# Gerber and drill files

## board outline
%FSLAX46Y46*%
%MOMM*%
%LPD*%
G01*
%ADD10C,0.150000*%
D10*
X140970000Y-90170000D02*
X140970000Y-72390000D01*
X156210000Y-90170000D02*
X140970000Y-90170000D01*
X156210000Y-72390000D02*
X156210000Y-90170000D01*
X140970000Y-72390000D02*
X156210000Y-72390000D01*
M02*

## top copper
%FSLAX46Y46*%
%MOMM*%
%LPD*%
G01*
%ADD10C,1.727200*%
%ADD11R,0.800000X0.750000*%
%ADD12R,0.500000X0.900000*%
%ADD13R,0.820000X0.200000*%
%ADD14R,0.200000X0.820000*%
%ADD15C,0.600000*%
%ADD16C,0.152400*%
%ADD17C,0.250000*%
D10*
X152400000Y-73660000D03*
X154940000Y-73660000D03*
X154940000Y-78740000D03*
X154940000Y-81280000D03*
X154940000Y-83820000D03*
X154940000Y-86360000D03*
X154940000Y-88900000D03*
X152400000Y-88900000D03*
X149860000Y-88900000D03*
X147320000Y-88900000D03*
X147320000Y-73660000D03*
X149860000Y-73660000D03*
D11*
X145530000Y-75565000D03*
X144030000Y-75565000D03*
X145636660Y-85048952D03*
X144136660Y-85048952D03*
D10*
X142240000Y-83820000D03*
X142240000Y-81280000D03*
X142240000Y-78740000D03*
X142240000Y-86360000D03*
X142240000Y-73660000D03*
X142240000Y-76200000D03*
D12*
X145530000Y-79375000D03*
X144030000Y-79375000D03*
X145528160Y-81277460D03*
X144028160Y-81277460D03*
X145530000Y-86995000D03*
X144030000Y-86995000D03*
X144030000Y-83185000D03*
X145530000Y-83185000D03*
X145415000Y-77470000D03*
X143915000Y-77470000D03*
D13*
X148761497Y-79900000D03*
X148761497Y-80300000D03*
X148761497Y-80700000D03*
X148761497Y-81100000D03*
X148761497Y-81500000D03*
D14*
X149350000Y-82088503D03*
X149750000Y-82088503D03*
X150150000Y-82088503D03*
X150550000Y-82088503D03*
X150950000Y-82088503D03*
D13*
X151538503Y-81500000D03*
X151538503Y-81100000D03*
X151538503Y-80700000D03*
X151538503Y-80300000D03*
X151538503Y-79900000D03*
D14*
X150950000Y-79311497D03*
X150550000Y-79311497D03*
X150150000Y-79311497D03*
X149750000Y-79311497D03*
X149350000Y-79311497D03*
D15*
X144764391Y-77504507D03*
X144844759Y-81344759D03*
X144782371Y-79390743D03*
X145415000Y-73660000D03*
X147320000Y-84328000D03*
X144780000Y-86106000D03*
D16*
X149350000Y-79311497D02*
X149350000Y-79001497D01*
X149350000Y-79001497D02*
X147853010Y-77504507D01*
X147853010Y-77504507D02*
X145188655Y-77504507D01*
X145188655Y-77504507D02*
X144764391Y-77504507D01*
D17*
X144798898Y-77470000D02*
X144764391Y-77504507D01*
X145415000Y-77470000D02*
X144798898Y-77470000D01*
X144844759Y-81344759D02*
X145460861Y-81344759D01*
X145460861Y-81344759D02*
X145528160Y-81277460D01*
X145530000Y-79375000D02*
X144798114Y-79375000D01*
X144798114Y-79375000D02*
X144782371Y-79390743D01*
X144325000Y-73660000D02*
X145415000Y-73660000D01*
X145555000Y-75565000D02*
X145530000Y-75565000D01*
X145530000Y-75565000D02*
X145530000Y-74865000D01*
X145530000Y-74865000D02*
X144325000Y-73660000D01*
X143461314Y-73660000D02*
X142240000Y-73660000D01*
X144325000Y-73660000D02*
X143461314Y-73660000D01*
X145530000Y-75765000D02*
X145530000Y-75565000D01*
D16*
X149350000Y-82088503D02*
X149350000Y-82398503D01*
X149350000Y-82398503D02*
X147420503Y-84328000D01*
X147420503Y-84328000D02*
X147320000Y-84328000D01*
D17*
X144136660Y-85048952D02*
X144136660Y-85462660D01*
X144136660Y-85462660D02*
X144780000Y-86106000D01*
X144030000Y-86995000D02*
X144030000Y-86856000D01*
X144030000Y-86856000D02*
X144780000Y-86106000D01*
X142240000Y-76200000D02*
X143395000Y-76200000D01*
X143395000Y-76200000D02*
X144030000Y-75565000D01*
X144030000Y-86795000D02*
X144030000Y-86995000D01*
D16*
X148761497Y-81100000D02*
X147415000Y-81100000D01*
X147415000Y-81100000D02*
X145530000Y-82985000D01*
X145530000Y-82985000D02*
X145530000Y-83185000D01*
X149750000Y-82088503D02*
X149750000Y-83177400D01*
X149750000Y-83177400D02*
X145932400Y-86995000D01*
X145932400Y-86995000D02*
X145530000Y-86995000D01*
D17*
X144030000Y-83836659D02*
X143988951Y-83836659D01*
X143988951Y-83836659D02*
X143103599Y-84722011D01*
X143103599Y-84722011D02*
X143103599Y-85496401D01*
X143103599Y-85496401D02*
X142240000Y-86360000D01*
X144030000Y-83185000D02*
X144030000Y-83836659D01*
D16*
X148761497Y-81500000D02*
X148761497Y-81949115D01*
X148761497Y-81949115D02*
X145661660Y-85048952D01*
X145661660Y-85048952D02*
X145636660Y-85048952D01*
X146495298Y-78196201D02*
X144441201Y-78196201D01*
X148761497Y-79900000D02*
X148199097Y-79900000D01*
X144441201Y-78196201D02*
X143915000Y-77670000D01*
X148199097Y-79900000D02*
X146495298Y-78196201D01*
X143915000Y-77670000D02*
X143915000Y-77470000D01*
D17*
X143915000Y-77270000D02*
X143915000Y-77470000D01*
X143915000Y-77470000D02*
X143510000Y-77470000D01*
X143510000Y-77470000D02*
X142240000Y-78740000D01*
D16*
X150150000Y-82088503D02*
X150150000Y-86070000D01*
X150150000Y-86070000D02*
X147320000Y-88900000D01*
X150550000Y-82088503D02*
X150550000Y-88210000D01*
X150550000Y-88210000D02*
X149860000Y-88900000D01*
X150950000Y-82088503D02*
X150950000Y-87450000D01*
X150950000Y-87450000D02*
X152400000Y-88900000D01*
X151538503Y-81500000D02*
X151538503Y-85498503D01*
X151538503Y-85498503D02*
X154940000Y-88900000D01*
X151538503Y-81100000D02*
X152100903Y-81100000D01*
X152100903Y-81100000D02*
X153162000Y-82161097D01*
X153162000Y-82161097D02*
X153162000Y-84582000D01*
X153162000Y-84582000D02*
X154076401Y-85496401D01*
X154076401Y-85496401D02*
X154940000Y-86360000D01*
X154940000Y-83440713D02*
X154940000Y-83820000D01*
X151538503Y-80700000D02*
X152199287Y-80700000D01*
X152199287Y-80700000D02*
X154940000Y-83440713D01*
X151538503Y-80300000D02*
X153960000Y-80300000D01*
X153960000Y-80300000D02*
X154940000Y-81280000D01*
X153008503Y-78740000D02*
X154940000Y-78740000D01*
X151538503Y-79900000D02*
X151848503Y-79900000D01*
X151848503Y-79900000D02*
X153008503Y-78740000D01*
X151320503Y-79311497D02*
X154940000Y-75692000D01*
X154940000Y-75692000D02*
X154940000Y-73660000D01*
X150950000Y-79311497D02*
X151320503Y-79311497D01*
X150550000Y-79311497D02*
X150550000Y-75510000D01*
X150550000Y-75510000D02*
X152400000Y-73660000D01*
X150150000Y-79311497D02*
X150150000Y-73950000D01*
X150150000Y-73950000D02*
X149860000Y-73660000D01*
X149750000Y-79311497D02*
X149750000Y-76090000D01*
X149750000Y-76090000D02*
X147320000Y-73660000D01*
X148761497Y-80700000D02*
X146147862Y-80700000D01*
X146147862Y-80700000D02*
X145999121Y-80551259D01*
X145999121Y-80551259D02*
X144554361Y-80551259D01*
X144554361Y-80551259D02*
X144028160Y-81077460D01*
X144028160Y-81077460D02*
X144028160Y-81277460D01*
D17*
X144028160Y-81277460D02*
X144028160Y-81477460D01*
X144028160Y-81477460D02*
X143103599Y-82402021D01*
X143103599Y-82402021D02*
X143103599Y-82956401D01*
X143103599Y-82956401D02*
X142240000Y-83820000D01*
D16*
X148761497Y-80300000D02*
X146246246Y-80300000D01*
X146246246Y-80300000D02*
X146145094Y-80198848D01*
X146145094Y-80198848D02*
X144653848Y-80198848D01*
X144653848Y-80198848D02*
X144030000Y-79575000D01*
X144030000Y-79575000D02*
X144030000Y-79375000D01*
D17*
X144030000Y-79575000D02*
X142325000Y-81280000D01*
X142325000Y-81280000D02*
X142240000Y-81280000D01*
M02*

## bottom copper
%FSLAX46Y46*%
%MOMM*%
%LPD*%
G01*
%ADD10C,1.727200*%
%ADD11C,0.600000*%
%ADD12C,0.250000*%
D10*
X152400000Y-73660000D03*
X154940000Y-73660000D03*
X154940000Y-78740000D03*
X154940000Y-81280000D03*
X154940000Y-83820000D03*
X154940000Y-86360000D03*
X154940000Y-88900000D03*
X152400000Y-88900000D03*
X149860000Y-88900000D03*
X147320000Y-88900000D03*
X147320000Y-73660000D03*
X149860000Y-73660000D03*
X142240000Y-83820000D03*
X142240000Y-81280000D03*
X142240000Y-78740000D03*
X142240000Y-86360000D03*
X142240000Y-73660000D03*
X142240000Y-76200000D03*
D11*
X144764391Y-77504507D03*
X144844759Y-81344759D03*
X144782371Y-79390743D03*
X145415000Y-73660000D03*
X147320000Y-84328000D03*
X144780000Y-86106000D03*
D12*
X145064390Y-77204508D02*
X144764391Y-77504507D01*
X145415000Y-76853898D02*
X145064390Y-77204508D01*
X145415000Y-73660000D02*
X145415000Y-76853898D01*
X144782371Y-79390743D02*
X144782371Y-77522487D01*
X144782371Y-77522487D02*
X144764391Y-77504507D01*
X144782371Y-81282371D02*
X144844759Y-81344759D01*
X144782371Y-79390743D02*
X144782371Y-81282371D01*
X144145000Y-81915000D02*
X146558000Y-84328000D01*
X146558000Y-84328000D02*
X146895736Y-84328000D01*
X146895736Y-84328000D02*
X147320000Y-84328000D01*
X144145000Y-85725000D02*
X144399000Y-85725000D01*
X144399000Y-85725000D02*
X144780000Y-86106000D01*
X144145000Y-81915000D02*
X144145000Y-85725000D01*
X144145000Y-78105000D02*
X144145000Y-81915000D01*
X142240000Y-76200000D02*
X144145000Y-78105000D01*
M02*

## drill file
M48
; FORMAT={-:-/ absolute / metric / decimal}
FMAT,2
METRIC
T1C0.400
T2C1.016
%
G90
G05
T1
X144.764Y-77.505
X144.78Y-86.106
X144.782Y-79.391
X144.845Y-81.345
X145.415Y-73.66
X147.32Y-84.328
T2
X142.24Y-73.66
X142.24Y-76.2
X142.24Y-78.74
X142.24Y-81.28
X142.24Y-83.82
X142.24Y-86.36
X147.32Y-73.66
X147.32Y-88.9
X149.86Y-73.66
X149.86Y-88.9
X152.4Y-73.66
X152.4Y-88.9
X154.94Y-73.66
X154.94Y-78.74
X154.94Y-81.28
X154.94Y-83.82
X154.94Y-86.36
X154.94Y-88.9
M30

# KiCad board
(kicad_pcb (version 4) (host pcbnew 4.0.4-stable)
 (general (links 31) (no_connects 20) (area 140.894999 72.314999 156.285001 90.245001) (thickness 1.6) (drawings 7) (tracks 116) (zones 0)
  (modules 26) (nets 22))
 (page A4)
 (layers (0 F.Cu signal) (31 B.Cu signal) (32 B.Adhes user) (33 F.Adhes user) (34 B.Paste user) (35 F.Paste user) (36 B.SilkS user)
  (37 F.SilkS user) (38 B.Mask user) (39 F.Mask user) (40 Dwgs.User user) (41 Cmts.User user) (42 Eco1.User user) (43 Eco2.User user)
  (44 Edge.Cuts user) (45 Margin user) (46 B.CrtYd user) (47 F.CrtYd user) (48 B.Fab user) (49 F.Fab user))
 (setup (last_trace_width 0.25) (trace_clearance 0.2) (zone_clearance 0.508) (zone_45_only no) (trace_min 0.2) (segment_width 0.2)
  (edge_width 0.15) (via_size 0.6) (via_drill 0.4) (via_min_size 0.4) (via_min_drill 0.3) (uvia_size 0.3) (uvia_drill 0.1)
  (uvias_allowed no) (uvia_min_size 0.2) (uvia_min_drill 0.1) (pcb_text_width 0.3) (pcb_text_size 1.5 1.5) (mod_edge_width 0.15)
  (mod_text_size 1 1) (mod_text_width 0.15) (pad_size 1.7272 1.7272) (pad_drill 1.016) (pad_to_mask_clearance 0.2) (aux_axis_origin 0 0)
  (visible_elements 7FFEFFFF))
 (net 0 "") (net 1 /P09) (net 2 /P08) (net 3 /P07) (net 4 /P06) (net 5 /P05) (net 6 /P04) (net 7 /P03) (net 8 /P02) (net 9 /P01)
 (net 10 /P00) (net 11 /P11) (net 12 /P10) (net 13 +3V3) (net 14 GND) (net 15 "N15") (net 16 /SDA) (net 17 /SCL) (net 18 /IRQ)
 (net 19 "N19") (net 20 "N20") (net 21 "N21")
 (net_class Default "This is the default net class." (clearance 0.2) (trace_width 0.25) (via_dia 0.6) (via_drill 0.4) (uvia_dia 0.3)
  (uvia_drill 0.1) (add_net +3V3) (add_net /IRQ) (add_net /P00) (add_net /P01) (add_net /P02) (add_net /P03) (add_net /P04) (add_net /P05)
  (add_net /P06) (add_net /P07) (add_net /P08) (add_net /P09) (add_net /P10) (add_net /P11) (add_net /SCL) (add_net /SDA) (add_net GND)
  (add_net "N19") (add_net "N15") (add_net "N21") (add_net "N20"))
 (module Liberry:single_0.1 (layer F.Cu) (at 152.4 73.66 90)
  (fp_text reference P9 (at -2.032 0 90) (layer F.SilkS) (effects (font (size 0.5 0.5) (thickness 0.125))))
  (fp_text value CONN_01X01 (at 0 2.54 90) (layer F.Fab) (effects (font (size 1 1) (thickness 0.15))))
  (pad 1 thru_hole circle (at 0 0 90) (size 1.7272 1.7272) (drill 1.016) (layers *.Cu *.Mask) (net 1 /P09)))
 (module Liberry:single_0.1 (layer F.Cu) (at 154.94 73.66 90)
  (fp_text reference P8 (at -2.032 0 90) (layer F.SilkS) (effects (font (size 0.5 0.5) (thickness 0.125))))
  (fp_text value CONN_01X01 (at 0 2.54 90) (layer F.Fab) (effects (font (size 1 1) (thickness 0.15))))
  (pad 1 thru_hole circle (at 0 0 90) (size 1.7272 1.7272) (drill 1.016) (layers *.Cu *.Mask) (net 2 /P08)))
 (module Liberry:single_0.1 (layer F.Cu) (at 154.94 78.74)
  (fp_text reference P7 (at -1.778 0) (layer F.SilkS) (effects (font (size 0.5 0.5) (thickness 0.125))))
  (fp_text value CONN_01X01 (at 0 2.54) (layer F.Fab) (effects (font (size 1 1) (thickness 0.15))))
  (pad 1 thru_hole circle (at 0 0) (size 1.7272 1.7272) (drill 1.016) (layers *.Cu *.Mask) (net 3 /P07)))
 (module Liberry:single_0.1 (layer F.Cu) (at 154.94 81.28 180)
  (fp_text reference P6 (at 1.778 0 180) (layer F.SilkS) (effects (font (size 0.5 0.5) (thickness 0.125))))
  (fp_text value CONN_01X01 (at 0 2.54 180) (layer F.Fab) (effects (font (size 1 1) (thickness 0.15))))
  (pad 1 thru_hole circle (at 0 0 180) (size 1.7272 1.7272) (drill 1.016) (layers *.Cu *.Mask) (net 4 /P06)))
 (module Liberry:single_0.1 (layer F.Cu) (at 154.94 83.82)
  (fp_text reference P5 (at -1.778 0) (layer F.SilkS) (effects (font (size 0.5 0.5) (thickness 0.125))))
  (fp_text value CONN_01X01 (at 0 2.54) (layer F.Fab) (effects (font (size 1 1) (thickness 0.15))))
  (pad 1 thru_hole circle (at 0 0) (size 1.7272 1.7272) (drill 1.016) (layers *.Cu *.Mask) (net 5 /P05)))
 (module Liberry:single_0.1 (layer F.Cu) (at 154.94 86.36)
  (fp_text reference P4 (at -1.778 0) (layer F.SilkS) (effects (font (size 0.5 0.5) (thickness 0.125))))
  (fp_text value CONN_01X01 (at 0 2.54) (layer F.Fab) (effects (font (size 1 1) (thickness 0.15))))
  (pad 1 thru_hole circle (at 0 0) (size 1.7272 1.7272) (drill 1.016) (layers *.Cu *.Mask) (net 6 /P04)))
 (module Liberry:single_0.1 (layer F.Cu) (at 154.94 88.9 270)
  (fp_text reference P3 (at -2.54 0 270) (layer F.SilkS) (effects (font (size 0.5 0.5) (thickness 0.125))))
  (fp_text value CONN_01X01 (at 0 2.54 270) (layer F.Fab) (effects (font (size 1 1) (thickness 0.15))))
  (pad 1 thru_hole circle (at 0 0 270) (size 1.7272 1.7272) (drill 1.016) (layers *.Cu *.Mask) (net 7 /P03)))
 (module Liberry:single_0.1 (layer F.Cu) (at 152.4 88.9 270)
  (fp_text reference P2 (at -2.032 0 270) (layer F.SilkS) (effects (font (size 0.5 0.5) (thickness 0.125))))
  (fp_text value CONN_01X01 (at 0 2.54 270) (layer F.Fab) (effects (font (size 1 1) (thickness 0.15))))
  (pad 1 thru_hole circle (at 0 0 270) (size 1.7272 1.7272) (drill 1.016) (layers *.Cu *.Mask) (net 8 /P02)))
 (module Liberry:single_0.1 (layer F.Cu) (at 149.86 88.9 270)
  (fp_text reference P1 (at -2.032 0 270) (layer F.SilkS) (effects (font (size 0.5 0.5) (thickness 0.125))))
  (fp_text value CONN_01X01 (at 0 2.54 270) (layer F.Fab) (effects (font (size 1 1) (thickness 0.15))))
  (pad 1 thru_hole circle (at 0 0 270) (size 1.7272 1.7272) (drill 1.016) (layers *.Cu *.Mask) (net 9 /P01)))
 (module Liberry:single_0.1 (layer F.Cu) (at 147.32 88.9 270)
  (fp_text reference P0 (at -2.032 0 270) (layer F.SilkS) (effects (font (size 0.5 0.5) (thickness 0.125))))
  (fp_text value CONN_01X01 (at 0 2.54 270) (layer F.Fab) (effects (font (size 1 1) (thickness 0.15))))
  (pad 1 thru_hole circle (at 0 0 270) (size 1.7272 1.7272) (drill 1.016) (layers *.Cu *.Mask) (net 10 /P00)))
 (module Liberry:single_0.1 (layer F.Cu) (at 147.32 73.66 90)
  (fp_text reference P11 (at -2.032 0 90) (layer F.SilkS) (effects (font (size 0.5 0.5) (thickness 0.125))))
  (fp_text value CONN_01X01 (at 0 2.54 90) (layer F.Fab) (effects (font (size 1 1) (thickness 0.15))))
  (pad 1 thru_hole circle (at 0 0 90) (size 1.7272 1.7272) (drill 1.016) (layers *.Cu *.Mask) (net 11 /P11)))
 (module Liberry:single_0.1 (layer F.Cu) (at 149.86 73.66 90)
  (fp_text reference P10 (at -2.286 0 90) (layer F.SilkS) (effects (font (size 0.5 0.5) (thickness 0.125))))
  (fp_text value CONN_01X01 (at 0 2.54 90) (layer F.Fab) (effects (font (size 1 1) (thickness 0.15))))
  (pad 1 thru_hole circle (at 0 0 90) (size 1.7272 1.7272) (drill 1.016) (layers *.Cu *.Mask) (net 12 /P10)))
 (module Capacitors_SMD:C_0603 (layer F.Cu) (at 144.78 75.565 180)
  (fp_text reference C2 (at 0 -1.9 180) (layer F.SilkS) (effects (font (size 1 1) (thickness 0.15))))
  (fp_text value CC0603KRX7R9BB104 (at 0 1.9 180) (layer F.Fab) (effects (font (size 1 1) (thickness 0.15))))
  (pad 1 smd rect (at -0.75 0 180) (size 0.8 0.75) (layers F.Cu F.Paste F.Mask) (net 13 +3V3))
  (pad 2 smd rect (at 0.75 0 180) (size 0.8 0.75) (layers F.Cu F.Paste F.Mask) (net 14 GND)))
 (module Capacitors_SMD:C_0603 (layer F.Cu) (at 144.88666 85.048952 180)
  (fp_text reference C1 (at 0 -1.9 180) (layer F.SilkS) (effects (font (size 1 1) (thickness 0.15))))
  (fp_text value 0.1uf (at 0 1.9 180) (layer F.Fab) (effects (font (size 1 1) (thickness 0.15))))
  (pad 1 smd rect (at -0.75 0 180) (size 0.8 0.75) (layers F.Cu F.Paste F.Mask) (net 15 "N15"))
  (pad 2 smd rect (at 0.75 0 180) (size 0.8 0.75) (layers F.Cu F.Paste F.Mask) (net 14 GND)))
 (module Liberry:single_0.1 (layer F.Cu) (at 142.24 83.82)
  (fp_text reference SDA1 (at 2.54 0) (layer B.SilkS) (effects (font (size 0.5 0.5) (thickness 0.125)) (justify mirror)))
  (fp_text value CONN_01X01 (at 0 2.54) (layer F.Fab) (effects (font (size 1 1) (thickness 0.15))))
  (pad 1 thru_hole circle (at 0 0) (size 1.7272 1.7272) (drill 1.016) (layers *.Cu *.Mask) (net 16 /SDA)))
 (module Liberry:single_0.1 (layer F.Cu) (at 142.24 81.28)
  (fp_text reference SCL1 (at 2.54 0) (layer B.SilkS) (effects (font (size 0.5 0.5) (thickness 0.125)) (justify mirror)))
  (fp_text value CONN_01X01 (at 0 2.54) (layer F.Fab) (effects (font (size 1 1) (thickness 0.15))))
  (pad 1 thru_hole circle (at 0 0) (size 1.7272 1.7272) (drill 1.016) (layers *.Cu *.Mask) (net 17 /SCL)))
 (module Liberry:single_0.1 (layer F.Cu) (at 142.24 78.74)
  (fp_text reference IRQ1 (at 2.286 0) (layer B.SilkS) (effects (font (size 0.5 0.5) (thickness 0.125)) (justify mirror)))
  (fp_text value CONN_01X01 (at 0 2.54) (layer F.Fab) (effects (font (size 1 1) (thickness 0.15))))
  (pad 1 thru_hole circle (at 0 0) (size 1.7272 1.7272) (drill 1.016) (layers *.Cu *.Mask) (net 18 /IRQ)))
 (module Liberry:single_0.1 (layer F.Cu) (at 142.24 86.36)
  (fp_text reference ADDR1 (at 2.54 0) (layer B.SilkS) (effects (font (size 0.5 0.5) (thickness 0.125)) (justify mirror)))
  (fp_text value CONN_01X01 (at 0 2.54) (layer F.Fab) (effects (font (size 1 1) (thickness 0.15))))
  (pad 1 thru_hole circle (at 0 0) (size 1.7272 1.7272) (drill 1.016) (layers *.Cu *.Mask) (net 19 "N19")))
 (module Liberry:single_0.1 (layer F.Cu) (at 142.24 73.66)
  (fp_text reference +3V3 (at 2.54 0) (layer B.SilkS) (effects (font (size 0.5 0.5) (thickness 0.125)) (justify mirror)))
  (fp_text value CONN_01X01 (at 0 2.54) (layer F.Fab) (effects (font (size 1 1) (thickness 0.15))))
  (pad 1 thru_hole circle (at 0 0) (size 1.7272 1.7272) (drill 1.016) (layers *.Cu *.Mask) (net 13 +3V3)))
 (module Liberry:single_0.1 (layer F.Cu) (at 142.24 76.2)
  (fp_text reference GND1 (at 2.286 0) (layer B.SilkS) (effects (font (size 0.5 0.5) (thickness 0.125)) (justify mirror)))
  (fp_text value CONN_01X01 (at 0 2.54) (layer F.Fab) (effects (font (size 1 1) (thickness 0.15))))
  (pad 1 thru_hole circle (at 0 0) (size 1.7272 1.7272) (drill 1.016) (layers *.Cu *.Mask) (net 14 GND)))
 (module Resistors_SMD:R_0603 (layer F.Cu) (at 144.78 79.375 180)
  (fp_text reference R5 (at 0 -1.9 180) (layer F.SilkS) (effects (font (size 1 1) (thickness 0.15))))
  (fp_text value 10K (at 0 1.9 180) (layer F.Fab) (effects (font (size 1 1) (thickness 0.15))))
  (pad 1 smd rect (at -0.75 0 180) (size 0.5 0.9) (layers F.Cu F.Paste F.Mask) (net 13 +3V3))
  (pad 2 smd rect (at 0.75 0 180) (size 0.5 0.9) (layers F.Cu F.Paste F.Mask) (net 17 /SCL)))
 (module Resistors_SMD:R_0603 (layer F.Cu) (at 144.77816 81.27746 180)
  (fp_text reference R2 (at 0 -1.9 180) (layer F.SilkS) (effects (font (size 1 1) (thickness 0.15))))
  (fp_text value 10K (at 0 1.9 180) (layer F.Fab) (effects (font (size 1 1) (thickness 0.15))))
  (pad 1 smd rect (at -0.75 0 180) (size 0.5 0.9) (layers F.Cu F.Paste F.Mask) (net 13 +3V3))
  (pad 2 smd rect (at 0.75 0 180) (size 0.5 0.9) (layers F.Cu F.Paste F.Mask) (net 16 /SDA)))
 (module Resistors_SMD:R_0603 (layer F.Cu) (at 144.78 86.995 180)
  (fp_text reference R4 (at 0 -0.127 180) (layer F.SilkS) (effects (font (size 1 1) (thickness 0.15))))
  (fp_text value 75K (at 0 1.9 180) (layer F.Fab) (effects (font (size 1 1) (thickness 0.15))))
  (pad 1 smd rect (at -0.75 0 180) (size 0.5 0.9) (layers F.Cu F.Paste F.Mask) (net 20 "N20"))
  (pad 2 smd rect (at 0.75 0 180) (size 0.5 0.9) (layers F.Cu F.Paste F.Mask) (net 14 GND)))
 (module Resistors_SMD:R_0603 (layer F.Cu) (at 144.78 83.185)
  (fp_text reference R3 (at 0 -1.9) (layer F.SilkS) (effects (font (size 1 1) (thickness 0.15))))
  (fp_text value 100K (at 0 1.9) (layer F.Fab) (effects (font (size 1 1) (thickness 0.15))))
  (pad 1 smd rect (at -0.75 0) (size 0.5 0.9) (layers F.Cu F.Paste F.Mask) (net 19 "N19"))
  (pad 2 smd rect (at 0.75 0) (size 0.5 0.9) (layers F.Cu F.Paste F.Mask) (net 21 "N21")))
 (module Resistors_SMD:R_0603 (layer F.Cu) (at 144.665 77.47 180)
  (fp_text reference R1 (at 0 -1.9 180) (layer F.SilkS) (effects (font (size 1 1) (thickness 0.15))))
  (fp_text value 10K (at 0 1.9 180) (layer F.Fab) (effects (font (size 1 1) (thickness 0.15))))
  (pad 1 smd rect (at -0.75 0 180) (size 0.5 0.9) (layers F.Cu F.Paste F.Mask) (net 13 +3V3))
  (pad 2 smd rect (at 0.75 0 180) (size 0.5 0.9) (layers F.Cu F.Paste F.Mask) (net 18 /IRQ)))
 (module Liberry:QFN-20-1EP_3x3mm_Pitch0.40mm (layer F.Cu) (at 150.15 80.7)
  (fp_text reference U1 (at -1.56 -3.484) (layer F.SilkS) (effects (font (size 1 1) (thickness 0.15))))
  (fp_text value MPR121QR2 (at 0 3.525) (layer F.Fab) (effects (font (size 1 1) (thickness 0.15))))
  (pad 1 smd rect (at -1.388503 -0.8) (size 0.82 0.2) (layers F.Cu F.Paste F.Mask) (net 18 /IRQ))
  (pad 2 smd rect (at -1.388503 -0.4) (size 0.82 0.2) (layers F.Cu F.Paste F.Mask) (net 17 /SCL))
  (pad 3 smd rect (at -1.388503 0) (size 0.82 0.2) (layers F.Cu F.Paste F.Mask) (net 16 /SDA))
  (pad 4 smd rect (at -1.388503 0.4) (size 0.82 0.2) (layers F.Cu F.Paste F.Mask) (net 21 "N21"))
  (pad 5 smd rect (at -1.388503 0.8) (size 0.82 0.2) (layers F.Cu F.Paste F.Mask) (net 15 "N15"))
  (pad 6 smd rect (at -0.8 1.388503 90) (size 0.82 0.2) (layers F.Cu F.Paste F.Mask) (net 14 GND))
  (pad 7 smd rect (at -0.4 1.388503 90) (size 0.82 0.2) (layers F.Cu F.Paste F.Mask) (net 20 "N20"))
  (pad 8 smd rect (at 0 1.388503 90) (size 0.82 0.2) (layers F.Cu F.Paste F.Mask) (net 10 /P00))
  (pad 9 smd rect (at 0.4 1.388503 90) (size 0.82 0.2) (layers F.Cu F.Paste F.Mask) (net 9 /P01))
  (pad 10 smd rect (at 0.8 1.388503 90) (size 0.82 0.2) (layers F.Cu F.Paste F.Mask) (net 8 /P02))
  (pad 11 smd rect (at 1.388503 0.8) (size 0.82 0.2) (layers F.Cu F.Paste F.Mask) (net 7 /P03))
  (pad 12 smd rect (at 1.388503 0.4) (size 0.82 0.2) (layers F.Cu F.Paste F.Mask) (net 6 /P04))
  (pad 13 smd rect (at 1.388503 0) (size 0.82 0.2) (layers F.Cu F.Paste F.Mask) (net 5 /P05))
  (pad 14 smd rect (at 1.388503 -0.4) (size 0.82 0.2) (layers F.Cu F.Paste F.Mask) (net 4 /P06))
  (pad 15 smd rect (at 1.388503 -0.8) (size 0.82 0.2) (layers F.Cu F.Paste F.Mask) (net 3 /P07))
  (pad 16 smd rect (at 0.8 -1.388503 90) (size 0.82 0.2) (layers F.Cu F.Paste F.Mask) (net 2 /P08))
  (pad 17 smd rect (at 0.4 -1.388503 90) (size 0.82 0.2) (layers F.Cu F.Paste F.Mask) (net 1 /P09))
  (pad 18 smd rect (at 0 -1.388503 90) (size 0.82 0.2) (layers F.Cu F.Paste F.Mask) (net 12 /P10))
  (pad 19 smd rect (at -0.4 -1.388503 90) (size 0.82 0.2) (layers F.Cu F.Paste F.Mask) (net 11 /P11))
  (pad 20 smd rect (at -0.8 -1.388503 90) (size 0.82 0.2) (layers F.Cu F.Paste F.Mask) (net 13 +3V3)))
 (gr_line (start 140.97 90.17) (end 140.97 72.39) (layer Edge.Cuts) (width 0.15))
 (gr_line (start 156.21 90.17) (end 140.97 90.17) (layer Edge.Cuts) (width 0.15))
 (gr_line (start 156.21 72.39) (end 156.21 90.17) (layer Edge.Cuts) (width 0.15))
 (gr_line (start 140.97 72.39) (end 156.21 72.39) (layer Edge.Cuts) (width 0.15))
 (segment (start 149.35 79.311497) (end 149.35 79.001497) (width 0.1524) (layer F.Cu) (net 13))
 (segment (start 149.35 79.001497) (end 147.85301 77.504507) (width 0.1524) (layer F.Cu) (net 13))
 (segment (start 147.85301 77.504507) (end 145.188655 77.504507) (width 0.1524) (layer F.Cu) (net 13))
 (segment (start 145.188655 77.504507) (end 144.764391 77.504507) (width 0.1524) (layer F.Cu) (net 13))
 (segment (start 145.06439 77.204508) (end 144.764391 77.504507) (width 0.25) (layer B.Cu) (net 13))
 (segment (start 145.415 76.853898) (end 145.06439 77.204508) (width 0.25) (layer B.Cu) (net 13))
 (segment (start 145.415 73.66) (end 145.415 76.853898) (width 0.25) (layer B.Cu) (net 13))
 (segment (start 144.798898 77.47) (end 144.764391 77.504507) (width 0.25) (layer F.Cu) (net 13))
 (segment (start 145.415 77.47) (end 144.798898 77.47) (width 0.25) (layer F.Cu) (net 13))
 (segment (start 144.782371 79.390743) (end 144.782371 77.522487) (width 0.25) (layer B.Cu) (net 13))
 (via (at 144.764391 77.504507) (size 0.6) (drill 0.4) (layers F.Cu B.Cu) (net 13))
 (segment (start 144.782371 77.522487) (end 144.764391 77.504507) (width 0.25) (layer B.Cu) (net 13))
 (segment (start 144.844759 81.344759) (end 145.460861 81.344759) (width 0.25) (layer F.Cu) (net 13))
 (segment (start 145.460861 81.344759) (end 145.52816 81.27746) (width 0.25) (layer F.Cu) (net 13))
 (segment (start 144.782371 81.282371) (end 144.844759 81.344759) (width 0.25) (layer B.Cu) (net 13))
 (segment (start 144.782371 79.390743) (end 144.782371 81.282371) (width 0.25) (layer B.Cu) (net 13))
 (via (at 144.844759 81.344759) (size 0.6) (drill 0.4) (layers F.Cu B.Cu) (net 13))
 (segment (start 145.53 79.375) (end 144.798114 79.375) (width 0.25) (layer F.Cu) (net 13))
 (segment (start 144.798114 79.375) (end 144.782371 79.390743) (width 0.25) (layer F.Cu) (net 13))
 (via (at 144.782371 79.390743) (size 0.6) (drill 0.4) (layers F.Cu B.Cu) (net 13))
 (segment (start 144.325 73.66) (end 145.415 73.66) (width 0.25) (layer F.Cu) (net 13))
 (via (at 145.415 73.66) (size 0.6) (drill 0.4) (layers F.Cu B.Cu) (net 13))
 (segment (start 145.555 75.565) (end 145.53 75.565) (width 0.25) (layer F.Cu) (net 13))
 (segment (start 145.53 75.565) (end 145.53 74.865) (width 0.25) (layer F.Cu) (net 13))
 (segment (start 145.53 74.865) (end 144.325 73.66) (width 0.25) (layer F.Cu) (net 13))
 (segment (start 143.461314 73.66) (end 142.24 73.66) (width 0.25) (layer F.Cu) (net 13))
 (segment (start 144.325 73.66) (end 143.461314 73.66) (width 0.25) (layer F.Cu) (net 13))
 (segment (start 145.53 75.765) (end 145.53 75.565) (width 0.25) (layer F.Cu) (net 13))
 (segment (start 149.35 82.088503) (end 149.35 82.398503) (width 0.1524) (layer F.Cu) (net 14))
 (segment (start 149.35 82.398503) (end 147.420503 84.328) (width 0.1524) (layer F.Cu) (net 14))
 (segment (start 147.420503 84.328) (end 147.32 84.328) (width 0.1524) (layer F.Cu) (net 14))
 (segment (start 144.145 81.915) (end 146.558 84.328) (width 0.25) (layer B.Cu) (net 14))
 (segment (start 146.558 84.328) (end 146.895736 84.328) (width 0.25) (layer B.Cu) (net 14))
 (segment (start 146.895736 84.328) (end 147.32 84.328) (width 0.25) (layer B.Cu) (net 14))
 (via (at 147.32 84.328) (size 0.6) (drill 0.4) (layers F.Cu B.Cu) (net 14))
 (segment (start 144.13666 85.048952) (end 144.13666 85.46266) (width 0.25) (layer F.Cu) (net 14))
 (segment (start 144.13666 85.46266) (end 144.78 86.106) (width 0.25) (layer F.Cu) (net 14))
 (segment (start 144.03 86.995) (end 144.03 86.856) (width 0.25) (layer F.Cu) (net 14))
 (segment (start 144.03 86.856) (end 144.78 86.106) (width 0.25) (layer F.Cu) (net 14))
 (segment (start 144.145 85.725) (end 144.399 85.725) (width 0.25) (layer B.Cu) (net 14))
 (segment (start 144.399 85.725) (end 144.78 86.106) (width 0.25) (layer B.Cu) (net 14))
 (segment (start 144.145 81.915) (end 144.145 85.725) (width 0.25) (layer B.Cu) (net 14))
 (via (at 144.78 86.106) (size 0.6) (drill 0.4) (layers F.Cu B.Cu) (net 14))
 (segment (start 144.145 78.105) (end 144.145 81.915) (width 0.25) (layer B.Cu) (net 14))
 (segment (start 142.24 76.2) (end 144.145 78.105) (width 0.25) (layer B.Cu) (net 14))
 (segment (start 142.24 76.2) (end 143.395 76.2) (width 0.25) (layer F.Cu) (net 14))
 (segment (start 143.395 76.2) (end 144.03 75.565) (width 0.25) (layer F.Cu) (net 14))
 (segment (start 144.03 86.795) (end 144.03 86.995) (width 0.25) (layer F.Cu) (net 14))
 (segment (start 148.761497 81.1) (end 147.415 81.1) (width 0.1524) (layer F.Cu) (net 21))
 (segment (start 147.415 81.1) (end 145.53 82.985) (width 0.1524) (layer F.Cu) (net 21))
 (segment (start 145.53 82.985) (end 145.53 83.185) (width 0.1524) (layer F.Cu) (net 21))
 (segment (start 149.75 82.088503) (end 149.75 83.1774) (width 0.1524) (layer F.Cu) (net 20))
 (segment (start 149.75 83.1774) (end 145.9324 86.995) (width 0.1524) (layer F.Cu) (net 20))
 (segment (start 145.9324 86.995) (end 145.53 86.995) (width 0.1524) (layer F.Cu) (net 20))
 (segment (start 144.03 83.836659) (end 143.988951 83.836659) (width 0.25) (layer F.Cu) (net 19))
 (segment (start 143.988951 83.836659) (end 143.103599 84.722011) (width 0.25) (layer F.Cu) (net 19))
 (segment (start 143.103599 84.722011) (end 143.103599 85.496401) (width 0.25) (layer F.Cu) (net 19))
 (segment (start 143.103599 85.496401) (end 142.24 86.36) (width 0.25) (layer F.Cu) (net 19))
 (segment (start 144.03 83.185) (end 144.03 83.836659) (width 0.25) (layer F.Cu) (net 19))
 (segment (start 148.761497 81.5) (end 148.761497 81.949115) (width 0.1524) (layer F.Cu) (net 15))
 (segment (start 148.761497 81.949115) (end 145.66166 85.048952) (width 0.1524) (layer F.Cu) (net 15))
 (segment (start 145.66166 85.048952) (end 145.63666 85.048952) (width 0.1524) (layer F.Cu) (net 15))
 (segment (start 146.495298 78.196201) (end 144.441201 78.196201) (width 0.1524) (layer F.Cu) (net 18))
 (segment (start 148.761497 79.9) (end 148.199097 79.9) (width 0.1524) (layer F.Cu) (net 18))
 (segment (start 144.441201 78.196201) (end 143.915 77.67) (width 0.1524) (layer F.Cu) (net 18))
 (segment (start 148.199097 79.9) (end 146.495298 78.196201) (width 0.1524) (layer F.Cu) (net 18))
 (segment (start 143.915 77.67) (end 143.915 77.47) (width 0.1524) (layer F.Cu) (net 18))
 (segment (start 143.915 77.27) (end 143.915 77.47) (width 0.25) (layer F.Cu) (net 18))
 (segment (start 143.915 77.47) (end 143.51 77.47) (width 0.25) (layer F.Cu) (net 18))
 (segment (start 143.51 77.47) (end 142.24 78.74) (width 0.25) (layer F.Cu) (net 18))
 (segment (start 150.15 82.088503) (end 150.15 86.07) (width 0.1524) (layer F.Cu) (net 10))
 (segment (start 150.15 86.07) (end 147.32 88.9) (width 0.1524) (layer F.Cu) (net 10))
 (segment (start 150.55 82.088503) (end 150.55 88.21) (width 0.1524) (layer F.Cu) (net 9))
 (segment (start 150.55 88.21) (end 149.86 88.9) (width 0.1524) (layer F.Cu) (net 9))
 (segment (start 150.95 82.088503) (end 150.95 87.45) (width 0.1524) (layer F.Cu) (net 8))
 (segment (start 150.95 87.45) (end 152.4 88.9) (width 0.1524) (layer F.Cu) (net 8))
 (segment (start 151.538503 81.5) (end 151.538503 85.498503) (width 0.1524) (layer F.Cu) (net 7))
 (segment (start 151.538503 85.498503) (end 154.94 88.9) (width 0.1524) (layer F.Cu) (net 7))
 (segment (start 151.538503 81.1) (end 152.100903 81.1) (width 0.1524) (layer F.Cu) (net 6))
 (segment (start 152.100903 81.1) (end 153.162 82.161097) (width 0.1524) (layer F.Cu) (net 6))
 (segment (start 153.162 82.161097) (end 153.162 84.582) (width 0.1524) (layer F.Cu) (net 6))
 (segment (start 153.162 84.582) (end 154.076401 85.496401) (width 0.1524) (layer F.Cu) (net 6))
 (segment (start 154.076401 85.496401) (end 154.94 86.36) (width 0.1524) (layer F.Cu) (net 6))
 (segment (start 154.94 83.440713) (end 154.94 83.82) (width 0.1524) (layer F.Cu) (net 5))
 (segment (start 151.538503 80.7) (end 152.199287 80.7) (width 0.1524) (layer F.Cu) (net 5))
 (segment (start 152.199287 80.7) (end 154.94 83.440713) (width 0.1524) (layer F.Cu) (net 5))
 (segment (start 151.538503 80.3) (end 153.96 80.3) (width 0.1524) (layer F.Cu) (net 4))
 (segment (start 153.96 80.3) (end 154.94 81.28) (width 0.1524) (layer F.Cu) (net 4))
 (segment (start 153.008503 78.74) (end 154.94 78.74) (width 0.1524) (layer F.Cu) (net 3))
 (segment (start 151.538503 79.9) (end 151.848503 79.9) (width 0.1524) (layer F.Cu) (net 3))
 (segment (start 151.848503 79.9) (end 153.008503 78.74) (width 0.1524) (layer F.Cu) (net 3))
 (segment (start 151.320503 79.311497) (end 154.94 75.692) (width 0.1524) (layer F.Cu) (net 2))
 (segment (start 154.94 75.692) (end 154.94 73.66) (width 0.1524) (layer F.Cu) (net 2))
 (segment (start 150.95 79.311497) (end 151.320503 79.311497) (width 0.1524) (layer F.Cu) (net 2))
 (segment (start 150.55 79.311497) (end 150.55 75.51) (width 0.1524) (layer F.Cu) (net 1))
 (segment (start 150.55 75.51) (end 152.4 73.66) (width 0.1524) (layer F.Cu) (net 1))
 (segment (start 150.15 79.311497) (end 150.15 73.95) (width 0.1524) (layer F.Cu) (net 12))
 (segment (start 150.15 73.95) (end 149.86 73.66) (width 0.1524) (layer F.Cu) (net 12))
 (segment (start 149.75 79.311497) (end 149.75 76.09) (width 0.1524) (layer F.Cu) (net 11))
 (segment (start 149.75 76.09) (end 147.32 73.66) (width 0.1524) (layer F.Cu) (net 11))
 (segment (start 148.761497 80.7) (end 146.147862 80.7) (width 0.1524) (layer F.Cu) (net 16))
 (segment (start 146.147862 80.7) (end 145.999121 80.551259) (width 0.1524) (layer F.Cu) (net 16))
 (segment (start 145.999121 80.551259) (end 144.554361 80.551259) (width 0.1524) (layer F.Cu) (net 16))
 (segment (start 144.554361 80.551259) (end 144.02816 81.07746) (width 0.1524) (layer F.Cu) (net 16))
 (segment (start 144.02816 81.07746) (end 144.02816 81.27746) (width 0.1524) (layer F.Cu) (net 16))
 (segment (start 144.02816 81.27746) (end 144.02816 81.47746) (width 0.25) (layer F.Cu) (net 16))
 (segment (start 144.02816 81.47746) (end 143.103599 82.402021) (width 0.25) (layer F.Cu) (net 16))
 (segment (start 143.103599 82.402021) (end 143.103599 82.956401) (width 0.25) (layer F.Cu) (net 16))
 (segment (start 143.103599 82.956401) (end 142.24 83.82) (width 0.25) (layer F.Cu) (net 16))
 (segment (start 148.761497 80.3) (end 146.246246 80.3) (width 0.1524) (layer F.Cu) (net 17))
 (segment (start 146.246246 80.3) (end 146.145094 80.198848) (width 0.1524) (layer F.Cu) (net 17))
 (segment (start 146.145094 80.198848) (end 144.653848 80.198848) (width 0.1524) (layer F.Cu) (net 17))
 (segment (start 144.653848 80.198848) (end 144.03 79.575) (width 0.1524) (layer F.Cu) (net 17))
 (segment (start 144.03 79.575) (end 144.03 79.375) (width 0.1524) (layer F.Cu) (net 17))
 (segment (start 144.03 79.575) (end 142.325 81.28) (width 0.25) (layer F.Cu) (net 17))
 (segment (start 142.325 81.28) (end 142.24 81.28) (width 0.25) (layer F.Cu) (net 17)))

